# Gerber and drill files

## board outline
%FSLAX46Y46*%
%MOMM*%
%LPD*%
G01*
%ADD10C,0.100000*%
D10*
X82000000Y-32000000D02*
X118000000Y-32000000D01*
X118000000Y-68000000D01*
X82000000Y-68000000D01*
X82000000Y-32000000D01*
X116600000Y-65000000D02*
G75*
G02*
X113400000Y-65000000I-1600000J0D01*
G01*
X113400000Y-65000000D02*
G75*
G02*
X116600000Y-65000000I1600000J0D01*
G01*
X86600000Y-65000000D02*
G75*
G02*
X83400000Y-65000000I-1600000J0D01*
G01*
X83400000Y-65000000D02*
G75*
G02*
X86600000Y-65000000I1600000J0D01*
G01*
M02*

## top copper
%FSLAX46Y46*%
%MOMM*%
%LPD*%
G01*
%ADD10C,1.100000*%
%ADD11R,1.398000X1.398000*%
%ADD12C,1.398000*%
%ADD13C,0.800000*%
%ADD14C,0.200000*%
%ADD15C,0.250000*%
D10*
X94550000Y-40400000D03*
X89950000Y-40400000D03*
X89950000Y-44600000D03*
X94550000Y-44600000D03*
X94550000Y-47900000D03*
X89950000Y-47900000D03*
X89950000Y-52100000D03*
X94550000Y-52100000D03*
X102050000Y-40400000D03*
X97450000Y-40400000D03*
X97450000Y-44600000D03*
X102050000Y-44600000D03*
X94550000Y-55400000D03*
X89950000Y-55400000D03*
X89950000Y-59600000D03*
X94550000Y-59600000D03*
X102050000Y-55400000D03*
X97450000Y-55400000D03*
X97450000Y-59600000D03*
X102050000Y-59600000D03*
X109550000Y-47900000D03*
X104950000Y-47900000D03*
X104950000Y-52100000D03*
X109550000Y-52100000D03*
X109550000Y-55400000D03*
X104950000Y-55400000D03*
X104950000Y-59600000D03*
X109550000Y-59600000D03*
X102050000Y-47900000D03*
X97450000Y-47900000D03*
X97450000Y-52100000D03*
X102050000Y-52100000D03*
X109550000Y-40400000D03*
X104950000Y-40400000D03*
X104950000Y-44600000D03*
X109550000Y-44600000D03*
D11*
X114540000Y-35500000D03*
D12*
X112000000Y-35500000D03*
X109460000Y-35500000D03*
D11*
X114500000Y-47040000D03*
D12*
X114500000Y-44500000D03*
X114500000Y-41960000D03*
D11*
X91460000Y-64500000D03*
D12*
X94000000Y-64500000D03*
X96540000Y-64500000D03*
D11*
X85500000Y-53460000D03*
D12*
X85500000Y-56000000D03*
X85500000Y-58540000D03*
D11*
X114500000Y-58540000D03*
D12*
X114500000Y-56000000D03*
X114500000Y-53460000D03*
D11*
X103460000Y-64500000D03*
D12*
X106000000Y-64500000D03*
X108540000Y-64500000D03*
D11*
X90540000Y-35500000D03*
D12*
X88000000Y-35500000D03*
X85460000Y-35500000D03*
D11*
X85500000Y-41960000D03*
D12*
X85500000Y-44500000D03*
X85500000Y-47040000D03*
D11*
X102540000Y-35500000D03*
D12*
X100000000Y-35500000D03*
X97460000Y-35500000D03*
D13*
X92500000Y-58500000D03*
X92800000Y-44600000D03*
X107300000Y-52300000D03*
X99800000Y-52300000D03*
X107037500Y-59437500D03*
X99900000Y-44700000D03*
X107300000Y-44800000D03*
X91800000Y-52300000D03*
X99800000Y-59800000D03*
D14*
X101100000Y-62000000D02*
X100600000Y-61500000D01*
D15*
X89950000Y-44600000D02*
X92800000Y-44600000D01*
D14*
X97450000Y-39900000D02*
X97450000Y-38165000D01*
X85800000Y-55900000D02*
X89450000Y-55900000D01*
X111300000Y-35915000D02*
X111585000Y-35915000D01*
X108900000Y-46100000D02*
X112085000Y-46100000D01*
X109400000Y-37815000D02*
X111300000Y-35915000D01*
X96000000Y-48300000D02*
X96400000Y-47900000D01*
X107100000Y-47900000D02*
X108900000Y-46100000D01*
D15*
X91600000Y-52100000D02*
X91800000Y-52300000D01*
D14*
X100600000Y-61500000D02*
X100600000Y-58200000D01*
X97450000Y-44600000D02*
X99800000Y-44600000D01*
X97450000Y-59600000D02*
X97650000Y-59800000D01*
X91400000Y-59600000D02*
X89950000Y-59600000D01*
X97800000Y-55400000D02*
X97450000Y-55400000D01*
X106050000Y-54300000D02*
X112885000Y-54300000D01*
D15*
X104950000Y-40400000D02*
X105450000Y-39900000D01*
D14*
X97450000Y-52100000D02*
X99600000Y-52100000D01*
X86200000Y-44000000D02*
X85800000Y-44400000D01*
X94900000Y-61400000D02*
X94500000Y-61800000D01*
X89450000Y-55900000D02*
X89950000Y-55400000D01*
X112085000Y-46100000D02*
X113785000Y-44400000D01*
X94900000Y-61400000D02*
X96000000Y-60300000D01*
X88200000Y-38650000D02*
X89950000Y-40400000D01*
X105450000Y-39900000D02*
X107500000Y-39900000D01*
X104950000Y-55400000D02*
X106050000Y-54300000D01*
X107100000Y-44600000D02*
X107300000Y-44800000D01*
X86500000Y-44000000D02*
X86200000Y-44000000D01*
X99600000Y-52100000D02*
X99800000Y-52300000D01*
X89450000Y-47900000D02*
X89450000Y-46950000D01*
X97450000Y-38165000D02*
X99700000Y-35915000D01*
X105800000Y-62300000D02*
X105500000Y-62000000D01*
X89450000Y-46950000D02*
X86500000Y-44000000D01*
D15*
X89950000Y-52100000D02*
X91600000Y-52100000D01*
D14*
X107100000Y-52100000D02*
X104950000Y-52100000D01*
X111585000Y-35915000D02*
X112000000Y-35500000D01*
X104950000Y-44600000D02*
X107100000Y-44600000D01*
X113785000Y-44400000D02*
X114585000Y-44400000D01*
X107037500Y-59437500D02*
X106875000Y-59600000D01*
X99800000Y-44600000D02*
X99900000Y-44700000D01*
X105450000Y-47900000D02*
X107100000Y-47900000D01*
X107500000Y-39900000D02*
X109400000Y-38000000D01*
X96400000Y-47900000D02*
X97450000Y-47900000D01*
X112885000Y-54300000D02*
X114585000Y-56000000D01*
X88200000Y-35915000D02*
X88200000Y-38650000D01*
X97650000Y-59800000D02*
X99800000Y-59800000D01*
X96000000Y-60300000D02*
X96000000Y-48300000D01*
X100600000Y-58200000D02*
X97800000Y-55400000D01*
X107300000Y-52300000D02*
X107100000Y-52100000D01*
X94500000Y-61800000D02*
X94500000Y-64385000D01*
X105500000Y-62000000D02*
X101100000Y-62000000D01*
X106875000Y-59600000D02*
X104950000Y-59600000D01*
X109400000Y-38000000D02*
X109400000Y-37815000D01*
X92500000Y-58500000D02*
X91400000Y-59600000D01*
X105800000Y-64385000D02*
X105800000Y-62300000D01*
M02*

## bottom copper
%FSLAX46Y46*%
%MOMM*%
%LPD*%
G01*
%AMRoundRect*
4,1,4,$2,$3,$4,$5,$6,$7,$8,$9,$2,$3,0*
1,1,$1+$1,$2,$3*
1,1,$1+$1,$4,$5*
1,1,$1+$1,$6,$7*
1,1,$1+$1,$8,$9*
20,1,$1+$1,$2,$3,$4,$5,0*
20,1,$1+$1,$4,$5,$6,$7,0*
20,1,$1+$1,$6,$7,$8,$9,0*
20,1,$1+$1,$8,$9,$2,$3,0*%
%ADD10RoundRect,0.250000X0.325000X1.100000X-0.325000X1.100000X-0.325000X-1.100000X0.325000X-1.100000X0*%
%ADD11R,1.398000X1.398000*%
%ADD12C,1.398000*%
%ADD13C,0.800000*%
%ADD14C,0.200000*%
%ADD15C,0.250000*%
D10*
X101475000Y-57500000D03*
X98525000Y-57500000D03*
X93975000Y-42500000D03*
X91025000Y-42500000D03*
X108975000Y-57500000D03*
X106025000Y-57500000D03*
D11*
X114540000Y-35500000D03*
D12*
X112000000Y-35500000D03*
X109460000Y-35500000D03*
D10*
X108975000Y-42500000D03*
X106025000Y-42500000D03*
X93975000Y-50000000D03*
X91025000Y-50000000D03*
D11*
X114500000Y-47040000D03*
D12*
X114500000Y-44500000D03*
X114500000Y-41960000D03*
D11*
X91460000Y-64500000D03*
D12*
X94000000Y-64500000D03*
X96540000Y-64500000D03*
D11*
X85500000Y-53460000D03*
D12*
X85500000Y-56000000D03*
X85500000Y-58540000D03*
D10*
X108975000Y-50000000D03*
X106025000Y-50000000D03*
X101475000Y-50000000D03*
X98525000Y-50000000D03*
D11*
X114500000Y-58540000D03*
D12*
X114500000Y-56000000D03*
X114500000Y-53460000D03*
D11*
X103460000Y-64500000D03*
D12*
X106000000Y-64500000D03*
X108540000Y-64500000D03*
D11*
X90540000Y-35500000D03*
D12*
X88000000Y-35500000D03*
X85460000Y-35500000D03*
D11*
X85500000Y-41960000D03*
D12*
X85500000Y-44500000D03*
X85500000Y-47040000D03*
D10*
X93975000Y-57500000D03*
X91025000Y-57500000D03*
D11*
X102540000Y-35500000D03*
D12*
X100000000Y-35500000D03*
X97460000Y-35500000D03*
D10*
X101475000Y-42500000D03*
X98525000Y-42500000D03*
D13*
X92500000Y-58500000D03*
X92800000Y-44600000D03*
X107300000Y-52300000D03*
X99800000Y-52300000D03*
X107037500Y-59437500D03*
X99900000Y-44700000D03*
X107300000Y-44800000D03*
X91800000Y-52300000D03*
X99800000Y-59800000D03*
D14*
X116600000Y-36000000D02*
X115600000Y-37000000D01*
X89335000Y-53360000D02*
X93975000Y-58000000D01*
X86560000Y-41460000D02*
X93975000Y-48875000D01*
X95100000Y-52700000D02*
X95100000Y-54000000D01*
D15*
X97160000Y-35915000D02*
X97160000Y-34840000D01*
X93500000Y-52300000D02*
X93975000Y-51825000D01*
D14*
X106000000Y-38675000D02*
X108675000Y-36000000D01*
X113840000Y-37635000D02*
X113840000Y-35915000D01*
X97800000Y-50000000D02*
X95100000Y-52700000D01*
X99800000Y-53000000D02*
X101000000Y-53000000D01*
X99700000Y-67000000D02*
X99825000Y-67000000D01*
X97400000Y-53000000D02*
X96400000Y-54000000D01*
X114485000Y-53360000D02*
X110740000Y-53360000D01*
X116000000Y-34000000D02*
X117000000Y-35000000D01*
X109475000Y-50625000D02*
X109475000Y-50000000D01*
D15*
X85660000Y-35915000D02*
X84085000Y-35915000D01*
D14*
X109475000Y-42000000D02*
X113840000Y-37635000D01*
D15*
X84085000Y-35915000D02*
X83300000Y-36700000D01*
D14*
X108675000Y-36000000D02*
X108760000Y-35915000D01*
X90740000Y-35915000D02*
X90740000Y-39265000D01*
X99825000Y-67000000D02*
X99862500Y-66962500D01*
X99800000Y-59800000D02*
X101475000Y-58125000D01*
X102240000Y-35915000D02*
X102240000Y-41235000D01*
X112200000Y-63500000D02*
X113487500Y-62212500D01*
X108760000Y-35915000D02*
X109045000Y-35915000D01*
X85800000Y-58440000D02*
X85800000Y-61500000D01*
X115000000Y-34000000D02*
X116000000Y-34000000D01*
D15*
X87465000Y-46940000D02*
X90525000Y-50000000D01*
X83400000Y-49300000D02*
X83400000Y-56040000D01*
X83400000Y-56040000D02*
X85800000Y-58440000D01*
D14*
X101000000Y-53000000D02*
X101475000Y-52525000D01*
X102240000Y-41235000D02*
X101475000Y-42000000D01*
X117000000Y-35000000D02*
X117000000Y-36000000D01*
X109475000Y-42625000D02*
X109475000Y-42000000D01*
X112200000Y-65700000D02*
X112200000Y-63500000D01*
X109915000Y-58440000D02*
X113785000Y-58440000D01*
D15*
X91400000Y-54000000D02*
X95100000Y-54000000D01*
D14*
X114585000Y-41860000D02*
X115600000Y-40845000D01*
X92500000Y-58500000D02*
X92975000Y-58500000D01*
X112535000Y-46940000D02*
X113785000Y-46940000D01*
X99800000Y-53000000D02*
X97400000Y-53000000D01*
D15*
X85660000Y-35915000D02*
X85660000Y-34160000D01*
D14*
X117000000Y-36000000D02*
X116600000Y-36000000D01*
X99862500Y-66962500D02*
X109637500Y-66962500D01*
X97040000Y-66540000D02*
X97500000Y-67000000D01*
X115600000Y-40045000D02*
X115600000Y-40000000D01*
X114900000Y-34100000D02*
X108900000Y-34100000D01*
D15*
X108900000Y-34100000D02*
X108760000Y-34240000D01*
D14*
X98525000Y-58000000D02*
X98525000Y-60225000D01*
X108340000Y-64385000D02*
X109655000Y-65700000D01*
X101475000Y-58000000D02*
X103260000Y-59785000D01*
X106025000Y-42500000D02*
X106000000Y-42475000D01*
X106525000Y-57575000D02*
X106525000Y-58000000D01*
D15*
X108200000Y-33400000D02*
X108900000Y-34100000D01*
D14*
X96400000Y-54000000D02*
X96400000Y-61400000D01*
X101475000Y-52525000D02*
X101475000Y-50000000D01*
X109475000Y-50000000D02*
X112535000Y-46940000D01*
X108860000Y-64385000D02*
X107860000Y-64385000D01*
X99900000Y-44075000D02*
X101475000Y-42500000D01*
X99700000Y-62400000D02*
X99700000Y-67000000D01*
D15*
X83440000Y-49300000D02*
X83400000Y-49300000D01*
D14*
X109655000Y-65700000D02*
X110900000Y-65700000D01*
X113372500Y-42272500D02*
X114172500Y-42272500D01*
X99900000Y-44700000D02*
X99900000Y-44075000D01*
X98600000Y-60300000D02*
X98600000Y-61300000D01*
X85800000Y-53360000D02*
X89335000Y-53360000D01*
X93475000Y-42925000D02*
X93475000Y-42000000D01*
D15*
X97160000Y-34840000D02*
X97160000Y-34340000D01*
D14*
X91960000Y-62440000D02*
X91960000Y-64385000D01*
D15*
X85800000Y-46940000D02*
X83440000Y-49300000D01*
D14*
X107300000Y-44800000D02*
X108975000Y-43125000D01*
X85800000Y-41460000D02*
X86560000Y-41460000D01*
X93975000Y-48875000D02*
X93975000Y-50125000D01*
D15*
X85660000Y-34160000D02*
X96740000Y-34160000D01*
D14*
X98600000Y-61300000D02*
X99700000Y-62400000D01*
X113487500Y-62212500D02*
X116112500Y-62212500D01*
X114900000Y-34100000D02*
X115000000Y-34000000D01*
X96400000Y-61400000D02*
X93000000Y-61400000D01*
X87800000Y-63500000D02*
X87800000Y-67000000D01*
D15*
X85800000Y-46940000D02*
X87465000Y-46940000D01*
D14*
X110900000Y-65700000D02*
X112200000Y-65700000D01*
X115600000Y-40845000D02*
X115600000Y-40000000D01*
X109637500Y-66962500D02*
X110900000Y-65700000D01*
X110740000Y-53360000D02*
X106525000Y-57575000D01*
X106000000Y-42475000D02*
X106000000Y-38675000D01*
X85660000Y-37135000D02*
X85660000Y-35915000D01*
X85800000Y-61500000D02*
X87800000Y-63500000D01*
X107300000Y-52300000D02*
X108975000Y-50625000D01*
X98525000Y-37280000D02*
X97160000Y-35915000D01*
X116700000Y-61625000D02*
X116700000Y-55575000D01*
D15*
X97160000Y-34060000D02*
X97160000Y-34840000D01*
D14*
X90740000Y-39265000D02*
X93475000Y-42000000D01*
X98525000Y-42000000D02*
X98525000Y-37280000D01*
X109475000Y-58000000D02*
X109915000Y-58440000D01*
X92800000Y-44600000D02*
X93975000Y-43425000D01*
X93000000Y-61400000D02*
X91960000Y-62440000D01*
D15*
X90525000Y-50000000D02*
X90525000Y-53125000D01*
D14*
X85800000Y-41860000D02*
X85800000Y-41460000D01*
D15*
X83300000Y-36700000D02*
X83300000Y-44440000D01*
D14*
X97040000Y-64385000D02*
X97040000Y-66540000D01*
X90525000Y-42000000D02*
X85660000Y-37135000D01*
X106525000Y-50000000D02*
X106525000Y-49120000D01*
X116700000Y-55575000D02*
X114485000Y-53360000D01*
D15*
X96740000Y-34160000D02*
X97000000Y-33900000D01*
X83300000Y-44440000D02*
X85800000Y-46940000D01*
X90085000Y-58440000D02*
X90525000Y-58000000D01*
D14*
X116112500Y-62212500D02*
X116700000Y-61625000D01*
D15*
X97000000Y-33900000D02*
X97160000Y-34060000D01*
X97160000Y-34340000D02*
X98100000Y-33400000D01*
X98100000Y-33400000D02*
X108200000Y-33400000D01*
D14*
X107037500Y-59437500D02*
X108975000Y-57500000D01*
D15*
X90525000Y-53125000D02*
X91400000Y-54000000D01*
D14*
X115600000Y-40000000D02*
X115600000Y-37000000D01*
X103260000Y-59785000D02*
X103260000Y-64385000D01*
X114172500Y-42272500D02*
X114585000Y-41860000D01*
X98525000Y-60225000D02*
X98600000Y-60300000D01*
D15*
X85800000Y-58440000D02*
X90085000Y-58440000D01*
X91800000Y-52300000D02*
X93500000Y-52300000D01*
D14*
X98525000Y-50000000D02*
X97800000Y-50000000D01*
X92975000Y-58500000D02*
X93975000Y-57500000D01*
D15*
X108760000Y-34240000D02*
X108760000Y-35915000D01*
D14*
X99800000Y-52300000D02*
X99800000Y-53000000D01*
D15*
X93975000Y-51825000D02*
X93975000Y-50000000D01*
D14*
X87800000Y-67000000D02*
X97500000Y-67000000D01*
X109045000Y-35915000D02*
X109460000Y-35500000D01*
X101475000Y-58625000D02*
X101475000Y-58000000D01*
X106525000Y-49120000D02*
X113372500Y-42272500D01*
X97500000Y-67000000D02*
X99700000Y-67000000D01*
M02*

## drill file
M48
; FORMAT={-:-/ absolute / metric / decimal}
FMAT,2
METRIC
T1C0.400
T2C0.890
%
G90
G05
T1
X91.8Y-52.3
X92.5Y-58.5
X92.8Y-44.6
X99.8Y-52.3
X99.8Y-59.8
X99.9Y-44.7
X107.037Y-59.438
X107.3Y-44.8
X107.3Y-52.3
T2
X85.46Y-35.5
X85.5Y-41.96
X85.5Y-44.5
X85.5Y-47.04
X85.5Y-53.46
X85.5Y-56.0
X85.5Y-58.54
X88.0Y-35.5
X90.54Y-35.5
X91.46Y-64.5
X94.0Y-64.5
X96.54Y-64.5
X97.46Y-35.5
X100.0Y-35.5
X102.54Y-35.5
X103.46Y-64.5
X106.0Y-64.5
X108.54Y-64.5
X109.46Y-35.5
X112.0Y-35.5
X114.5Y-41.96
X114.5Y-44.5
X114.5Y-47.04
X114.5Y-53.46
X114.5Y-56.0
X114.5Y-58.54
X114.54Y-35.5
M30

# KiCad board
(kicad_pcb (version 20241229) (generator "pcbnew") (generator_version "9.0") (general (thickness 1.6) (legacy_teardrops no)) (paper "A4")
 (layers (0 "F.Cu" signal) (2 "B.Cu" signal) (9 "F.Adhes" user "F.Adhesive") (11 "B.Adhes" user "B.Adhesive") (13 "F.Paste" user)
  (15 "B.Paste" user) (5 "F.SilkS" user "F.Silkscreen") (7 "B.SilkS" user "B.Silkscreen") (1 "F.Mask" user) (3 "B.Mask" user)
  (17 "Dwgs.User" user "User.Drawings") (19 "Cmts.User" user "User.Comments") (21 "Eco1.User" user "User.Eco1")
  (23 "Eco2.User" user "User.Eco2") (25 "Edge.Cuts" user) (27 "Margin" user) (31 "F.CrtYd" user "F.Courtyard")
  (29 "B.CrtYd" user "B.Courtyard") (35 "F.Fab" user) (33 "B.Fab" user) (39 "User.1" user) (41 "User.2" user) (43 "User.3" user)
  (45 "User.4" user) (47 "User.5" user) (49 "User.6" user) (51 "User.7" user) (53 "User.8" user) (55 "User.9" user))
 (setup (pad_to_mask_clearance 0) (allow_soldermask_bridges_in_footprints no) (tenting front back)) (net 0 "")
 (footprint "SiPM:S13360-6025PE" (layer "F.Cu") (at 92.5 42.5)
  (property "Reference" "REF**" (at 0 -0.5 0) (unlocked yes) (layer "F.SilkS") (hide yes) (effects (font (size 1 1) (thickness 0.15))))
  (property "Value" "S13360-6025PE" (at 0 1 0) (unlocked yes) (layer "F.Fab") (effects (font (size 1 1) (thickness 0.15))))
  (pad "1" smd circle (at 2.05 -2.1) (size 1.1 1.1) (layers "F.Cu" "F.Mask" "F.Paste"))
  (pad "2" smd circle (at -2.55 -2.1) (size 1.1 1.1) (layers "F.Cu" "F.Mask" "F.Paste"))
  (pad "3" smd circle (at -2.55 2.1) (size 1.1 1.1) (layers "F.Cu" "F.Mask" "F.Paste"))
  (pad "4" smd circle (at 2.05 2.1) (size 1.1 1.1) (layers "F.Cu" "F.Mask" "F.Paste")))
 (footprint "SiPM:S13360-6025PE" (layer "F.Cu") (at 92.5 50)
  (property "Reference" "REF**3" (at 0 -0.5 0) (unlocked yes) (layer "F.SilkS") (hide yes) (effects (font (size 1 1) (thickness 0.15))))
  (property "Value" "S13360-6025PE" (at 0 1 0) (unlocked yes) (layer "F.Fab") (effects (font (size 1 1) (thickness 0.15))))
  (pad "1" smd circle (at 2.05 -2.1) (size 1.1 1.1) (layers "F.Cu" "F.Mask" "F.Paste"))
  (pad "2" smd circle (at -2.55 -2.1) (size 1.1 1.1) (layers "F.Cu" "F.Mask" "F.Paste"))
  (pad "3" smd circle (at -2.55 2.1) (size 1.1 1.1) (layers "F.Cu" "F.Mask" "F.Paste"))
  (pad "4" smd circle (at 2.05 2.1) (size 1.1 1.1) (layers "F.Cu" "F.Mask" "F.Paste")))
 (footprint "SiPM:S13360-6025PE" (layer "F.Cu") (at 100 42.5)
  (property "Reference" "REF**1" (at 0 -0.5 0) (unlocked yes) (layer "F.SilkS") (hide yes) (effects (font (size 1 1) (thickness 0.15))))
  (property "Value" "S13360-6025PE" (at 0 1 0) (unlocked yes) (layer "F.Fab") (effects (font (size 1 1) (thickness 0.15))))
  (pad "1" smd circle (at 2.05 -2.1) (size 1.1 1.1) (layers "F.Cu" "F.Mask" "F.Paste"))
  (pad "2" smd circle (at -2.55 -2.1) (size 1.1 1.1) (layers "F.Cu" "F.Mask" "F.Paste"))
  (pad "3" smd circle (at -2.55 2.1) (size 1.1 1.1) (layers "F.Cu" "F.Mask" "F.Paste"))
  (pad "4" smd circle (at 2.05 2.1) (size 1.1 1.1) (layers "F.Cu" "F.Mask" "F.Paste")))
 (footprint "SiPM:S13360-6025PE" (layer "F.Cu") (at 92.5 57.5)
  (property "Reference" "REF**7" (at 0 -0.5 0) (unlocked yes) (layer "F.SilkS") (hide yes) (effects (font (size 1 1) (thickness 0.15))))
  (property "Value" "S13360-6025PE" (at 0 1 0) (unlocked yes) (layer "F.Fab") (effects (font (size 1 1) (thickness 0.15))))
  (pad "1" smd circle (at 2.05 -2.1) (size 1.1 1.1) (layers "F.Cu" "F.Mask" "F.Paste"))
  (pad "2" smd circle (at -2.55 -2.1) (size 1.1 1.1) (layers "F.Cu" "F.Mask" "F.Paste"))
  (pad "3" smd circle (at -2.55 2.1) (size 1.1 1.1) (layers "F.Cu" "F.Mask" "F.Paste"))
  (pad "4" smd circle (at 2.05 2.1) (size 1.1 1.1) (layers "F.Cu" "F.Mask" "F.Paste")))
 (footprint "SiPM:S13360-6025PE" (layer "F.Cu") (at 100 57.5)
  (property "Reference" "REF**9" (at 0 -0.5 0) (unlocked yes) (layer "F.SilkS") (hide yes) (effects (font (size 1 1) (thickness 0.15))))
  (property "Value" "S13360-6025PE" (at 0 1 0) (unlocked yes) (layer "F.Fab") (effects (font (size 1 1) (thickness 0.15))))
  (pad "1" smd circle (at 2.05 -2.1) (size 1.1 1.1) (layers "F.Cu" "F.Mask" "F.Paste"))
  (pad "2" smd circle (at -2.55 -2.1) (size 1.1 1.1) (layers "F.Cu" "F.Mask" "F.Paste"))
  (pad "3" smd circle (at -2.55 2.1) (size 1.1 1.1) (layers "F.Cu" "F.Mask" "F.Paste"))
  (pad "4" smd circle (at 2.05 2.1) (size 1.1 1.1) (layers "F.Cu" "F.Mask" "F.Paste")))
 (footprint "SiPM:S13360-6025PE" (layer "F.Cu") (at 107.5 50)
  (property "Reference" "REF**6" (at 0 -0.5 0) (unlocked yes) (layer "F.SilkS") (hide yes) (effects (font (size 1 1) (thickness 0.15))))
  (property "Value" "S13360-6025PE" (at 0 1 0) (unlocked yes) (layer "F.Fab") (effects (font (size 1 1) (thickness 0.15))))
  (pad "1" smd circle (at 2.05 -2.1) (size 1.1 1.1) (layers "F.Cu" "F.Mask" "F.Paste"))
  (pad "2" smd circle (at -2.55 -2.1) (size 1.1 1.1) (layers "F.Cu" "F.Mask" "F.Paste"))
  (pad "3" smd circle (at -2.55 2.1) (size 1.1 1.1) (layers "F.Cu" "F.Mask" "F.Paste"))
  (pad "4" smd circle (at 2.05 2.1) (size 1.1 1.1) (layers "F.Cu" "F.Mask" "F.Paste")))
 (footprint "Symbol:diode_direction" (layer "F.Cu") (at 87.3 41.8 90)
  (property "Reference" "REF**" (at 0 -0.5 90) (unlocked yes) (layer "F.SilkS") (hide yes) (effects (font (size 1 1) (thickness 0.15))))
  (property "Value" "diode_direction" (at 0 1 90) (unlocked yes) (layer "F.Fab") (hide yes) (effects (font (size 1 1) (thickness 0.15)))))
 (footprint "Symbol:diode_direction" (layer "F.Cu") (at 87.3 49.8 90)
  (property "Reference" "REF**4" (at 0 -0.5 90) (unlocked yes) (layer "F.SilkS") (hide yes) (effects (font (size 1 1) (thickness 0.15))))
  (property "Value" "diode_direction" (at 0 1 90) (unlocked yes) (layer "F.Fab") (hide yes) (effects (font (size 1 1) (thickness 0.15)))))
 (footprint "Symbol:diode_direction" (layer "F.Cu") (at 87.3 57.8 90)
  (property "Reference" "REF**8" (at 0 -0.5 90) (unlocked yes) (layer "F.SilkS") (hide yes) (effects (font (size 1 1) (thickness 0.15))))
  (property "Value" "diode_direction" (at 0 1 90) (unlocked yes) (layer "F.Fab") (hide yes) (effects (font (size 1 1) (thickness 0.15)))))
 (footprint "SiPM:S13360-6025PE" (layer "F.Cu") (at 107.5 57.5)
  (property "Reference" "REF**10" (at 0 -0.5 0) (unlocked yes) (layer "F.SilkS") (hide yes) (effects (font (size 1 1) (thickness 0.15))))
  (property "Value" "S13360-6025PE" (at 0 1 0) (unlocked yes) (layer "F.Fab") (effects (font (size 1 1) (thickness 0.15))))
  (pad "1" smd circle (at 2.05 -2.1) (size 1.1 1.1) (layers "F.Cu" "F.Mask" "F.Paste"))
  (pad "2" smd circle (at -2.55 -2.1) (size 1.1 1.1) (layers "F.Cu" "F.Mask" "F.Paste"))
  (pad "3" smd circle (at -2.55 2.1) (size 1.1 1.1) (layers "F.Cu" "F.Mask" "F.Paste"))
  (pad "4" smd circle (at 2.05 2.1) (size 1.1 1.1) (layers "F.Cu" "F.Mask" "F.Paste")))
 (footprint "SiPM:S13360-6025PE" (layer "F.Cu") (at 100 50)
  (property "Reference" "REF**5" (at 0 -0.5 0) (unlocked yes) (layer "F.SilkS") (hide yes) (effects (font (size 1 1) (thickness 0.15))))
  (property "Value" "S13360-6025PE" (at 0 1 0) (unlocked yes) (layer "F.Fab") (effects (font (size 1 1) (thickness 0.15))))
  (pad "1" smd circle (at 2.05 -2.1) (size 1.1 1.1) (layers "F.Cu" "F.Mask" "F.Paste"))
  (pad "2" smd circle (at -2.55 -2.1) (size 1.1 1.1) (layers "F.Cu" "F.Mask" "F.Paste"))
  (pad "3" smd circle (at -2.55 2.1) (size 1.1 1.1) (layers "F.Cu" "F.Mask" "F.Paste"))
  (pad "4" smd circle (at 2.05 2.1) (size 1.1 1.1) (layers "F.Cu" "F.Mask" "F.Paste")))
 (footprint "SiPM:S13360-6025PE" (layer "F.Cu") (at 107.5 42.5)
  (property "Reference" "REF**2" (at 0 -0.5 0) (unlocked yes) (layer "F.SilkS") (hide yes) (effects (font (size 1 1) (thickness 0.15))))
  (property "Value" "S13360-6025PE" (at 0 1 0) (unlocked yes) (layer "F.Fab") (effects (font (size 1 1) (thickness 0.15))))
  (pad "1" smd circle (at 2.05 -2.1) (size 1.1 1.1) (layers "F.Cu" "F.Mask" "F.Paste"))
  (pad "2" smd circle (at -2.55 -2.1) (size 1.1 1.1) (layers "F.Cu" "F.Mask" "F.Paste"))
  (pad "3" smd circle (at -2.55 2.1) (size 1.1 1.1) (layers "F.Cu" "F.Mask" "F.Paste"))
  (pad "4" smd circle (at 2.05 2.1) (size 1.1 1.1) (layers "F.Cu" "F.Mask" "F.Paste")))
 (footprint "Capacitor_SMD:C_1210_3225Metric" (layer "B.Cu") (at 100 57.5 180)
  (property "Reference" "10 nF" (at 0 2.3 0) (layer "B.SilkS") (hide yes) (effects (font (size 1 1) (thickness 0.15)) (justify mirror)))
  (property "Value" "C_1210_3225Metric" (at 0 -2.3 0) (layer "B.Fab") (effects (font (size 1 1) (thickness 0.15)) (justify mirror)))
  (pad "1" smd roundrect (at -1.475 0 180) (size 1.15 2.7) (layers "B.Cu" "B.Mask" "B.Paste") (roundrect_rratio 0.2173913043))
  (pad "2" smd roundrect (at 1.475 0 180) (size 1.15 2.7) (layers "B.Cu" "B.Mask" "B.Paste") (roundrect_rratio 0.2173913043)))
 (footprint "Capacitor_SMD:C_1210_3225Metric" (layer "B.Cu") (at 92.5 42.5 180)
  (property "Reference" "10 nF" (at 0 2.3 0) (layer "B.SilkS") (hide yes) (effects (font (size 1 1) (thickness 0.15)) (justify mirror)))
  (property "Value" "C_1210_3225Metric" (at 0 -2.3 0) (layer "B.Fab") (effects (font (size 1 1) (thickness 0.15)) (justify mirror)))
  (pad "1" smd roundrect (at -1.475 0 180) (size 1.15 2.7) (layers "B.Cu" "B.Mask" "B.Paste") (roundrect_rratio 0.2173913043))
  (pad "2" smd roundrect (at 1.475 0 180) (size 1.15 2.7) (layers "B.Cu" "B.Mask" "B.Paste") (roundrect_rratio 0.2173913043)))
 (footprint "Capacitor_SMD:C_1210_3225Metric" (layer "B.Cu") (at 107.5 57.5 180)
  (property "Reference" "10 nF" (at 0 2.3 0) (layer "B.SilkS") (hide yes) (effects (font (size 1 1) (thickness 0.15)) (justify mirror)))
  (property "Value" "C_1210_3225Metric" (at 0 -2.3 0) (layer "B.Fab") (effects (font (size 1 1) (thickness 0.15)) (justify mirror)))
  (pad "1" smd roundrect (at -1.475 0 180) (size 1.15 2.7) (layers "B.Cu" "B.Mask" "B.Paste") (roundrect_rratio 0.2173913043))
  (pad "2" smd roundrect (at 1.475 0 180) (size 1.15 2.7) (layers "B.Cu" "B.Mask" "B.Paste") (roundrect_rratio 0.2173913043)))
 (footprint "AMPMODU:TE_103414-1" (layer "B.Cu") (at 112 35.5 180)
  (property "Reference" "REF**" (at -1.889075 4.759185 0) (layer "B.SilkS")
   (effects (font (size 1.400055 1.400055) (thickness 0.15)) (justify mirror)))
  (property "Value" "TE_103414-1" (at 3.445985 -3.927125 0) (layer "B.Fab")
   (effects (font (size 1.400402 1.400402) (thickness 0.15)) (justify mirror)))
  (pad "1" thru_hole rect (at -2.54 0 180) (size 1.398 1.398) (drill 0.89) (layers "*.Cu" "*.Mask") (remove_unused_layers no)
   (solder_mask_margin 0.102))
  (pad "2" thru_hole circle (at 0 0 180) (size 1.398 1.398) (drill 0.89) (layers "*.Cu" "*.Mask") (remove_unused_layers no)
   (solder_mask_margin 0.102))
  (pad "3" thru_hole circle (at 2.54 0 180) (size 1.398 1.398) (drill 0.89) (layers "*.Cu" "*.Mask") (remove_unused_layers no)
   (solder_mask_margin 0.102)))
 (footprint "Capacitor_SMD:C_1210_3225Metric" (layer "B.Cu") (at 107.5 42.5 180)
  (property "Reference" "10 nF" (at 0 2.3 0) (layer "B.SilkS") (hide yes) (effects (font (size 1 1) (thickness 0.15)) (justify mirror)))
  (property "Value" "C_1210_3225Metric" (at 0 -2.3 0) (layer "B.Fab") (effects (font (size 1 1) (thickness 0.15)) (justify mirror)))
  (pad "1" smd roundrect (at -1.475 0 180) (size 1.15 2.7) (layers "B.Cu" "B.Mask" "B.Paste") (roundrect_rratio 0.2173913043))
  (pad "2" smd roundrect (at 1.475 0 180) (size 1.15 2.7) (layers "B.Cu" "B.Mask" "B.Paste") (roundrect_rratio 0.2173913043)))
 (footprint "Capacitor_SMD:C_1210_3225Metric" (layer "B.Cu") (at 92.5 50 180)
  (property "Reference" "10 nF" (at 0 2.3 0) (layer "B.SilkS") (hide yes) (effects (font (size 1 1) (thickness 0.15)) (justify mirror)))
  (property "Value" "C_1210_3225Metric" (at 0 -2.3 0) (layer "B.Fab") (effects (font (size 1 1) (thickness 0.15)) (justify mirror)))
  (pad "1" smd roundrect (at -1.475 0 180) (size 1.15 2.7) (layers "B.Cu" "B.Mask" "B.Paste") (roundrect_rratio 0.2173913043))
  (pad "2" smd roundrect (at 1.475 0 180) (size 1.15 2.7) (layers "B.Cu" "B.Mask" "B.Paste") (roundrect_rratio 0.2173913043)))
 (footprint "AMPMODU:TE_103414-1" (layer "B.Cu") (at 114.5 44.5 90)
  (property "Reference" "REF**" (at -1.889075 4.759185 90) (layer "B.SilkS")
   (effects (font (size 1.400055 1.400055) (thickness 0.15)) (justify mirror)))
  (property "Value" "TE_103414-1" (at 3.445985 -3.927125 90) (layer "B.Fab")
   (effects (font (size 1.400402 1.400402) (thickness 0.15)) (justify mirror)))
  (pad "1" thru_hole rect (at -2.54 0 90) (size 1.398 1.398) (drill 0.89) (layers "*.Cu" "*.Mask") (remove_unused_layers no)
   (solder_mask_margin 0.102))
  (pad "2" thru_hole circle (at 0 0 90) (size 1.398 1.398) (drill 0.89) (layers "*.Cu" "*.Mask") (remove_unused_layers no)
   (solder_mask_margin 0.102))
  (pad "3" thru_hole circle (at 2.54 0 90) (size 1.398 1.398) (drill 0.89) (layers "*.Cu" "*.Mask") (remove_unused_layers no)
   (solder_mask_margin 0.102)))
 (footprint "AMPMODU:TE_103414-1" (layer "B.Cu") (at 94 64.5)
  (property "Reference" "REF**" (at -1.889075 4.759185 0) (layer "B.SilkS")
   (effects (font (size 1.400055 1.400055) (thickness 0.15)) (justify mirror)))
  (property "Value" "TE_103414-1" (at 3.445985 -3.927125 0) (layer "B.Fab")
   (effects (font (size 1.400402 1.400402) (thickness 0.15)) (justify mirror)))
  (pad "1" thru_hole rect (at -2.54 0) (size 1.398 1.398) (drill 0.89) (layers "*.Cu" "*.Mask") (remove_unused_layers no)
   (solder_mask_margin 0.102))
  (pad "2" thru_hole circle (at 0 0) (size 1.398 1.398) (drill 0.89) (layers "*.Cu" "*.Mask") (remove_unused_layers no)
   (solder_mask_margin 0.102))
  (pad "3" thru_hole circle (at 2.54 0) (size 1.398 1.398) (drill 0.89) (layers "*.Cu" "*.Mask") (remove_unused_layers no)
   (solder_mask_margin 0.102)))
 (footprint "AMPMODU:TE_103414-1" (layer "B.Cu") (at 85.5 56 -90)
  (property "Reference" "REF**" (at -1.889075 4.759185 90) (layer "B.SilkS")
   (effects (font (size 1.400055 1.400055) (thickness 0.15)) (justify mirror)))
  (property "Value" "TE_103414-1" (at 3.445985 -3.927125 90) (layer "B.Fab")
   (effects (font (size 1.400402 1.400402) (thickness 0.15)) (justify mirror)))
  (pad "1" thru_hole rect (at -2.54 0 270) (size 1.398 1.398) (drill 0.89) (layers "*.Cu" "*.Mask") (remove_unused_layers no)
   (solder_mask_margin 0.102))
  (pad "2" thru_hole circle (at 0 0 270) (size 1.398 1.398) (drill 0.89) (layers "*.Cu" "*.Mask") (remove_unused_layers no)
   (solder_mask_margin 0.102))
  (pad "3" thru_hole circle (at 2.54 0 270) (size 1.398 1.398) (drill 0.89) (layers "*.Cu" "*.Mask") (remove_unused_layers no)
   (solder_mask_margin 0.102)))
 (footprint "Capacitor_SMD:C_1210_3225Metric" (layer "B.Cu") (at 107.5 50 180)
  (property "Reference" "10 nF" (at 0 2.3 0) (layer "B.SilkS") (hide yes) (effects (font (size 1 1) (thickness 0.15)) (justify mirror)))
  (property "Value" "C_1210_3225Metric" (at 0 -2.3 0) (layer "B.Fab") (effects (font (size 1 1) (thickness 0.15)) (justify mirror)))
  (pad "1" smd roundrect (at -1.475 0 180) (size 1.15 2.7) (layers "B.Cu" "B.Mask" "B.Paste") (roundrect_rratio 0.2173913043))
  (pad "2" smd roundrect (at 1.475 0 180) (size 1.15 2.7) (layers "B.Cu" "B.Mask" "B.Paste") (roundrect_rratio 0.2173913043)))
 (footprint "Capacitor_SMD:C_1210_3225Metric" (layer "B.Cu") (at 100 50 180)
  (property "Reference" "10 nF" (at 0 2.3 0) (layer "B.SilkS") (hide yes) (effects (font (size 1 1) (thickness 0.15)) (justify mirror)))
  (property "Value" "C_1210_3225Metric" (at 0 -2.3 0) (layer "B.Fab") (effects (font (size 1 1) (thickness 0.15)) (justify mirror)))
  (pad "1" smd roundrect (at -1.475 0 180) (size 1.15 2.7) (layers "B.Cu" "B.Mask" "B.Paste") (roundrect_rratio 0.2173913043))
  (pad "2" smd roundrect (at 1.475 0 180) (size 1.15 2.7) (layers "B.Cu" "B.Mask" "B.Paste") (roundrect_rratio 0.2173913043)))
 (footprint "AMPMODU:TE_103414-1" (layer "B.Cu") (at 114.5 56 90)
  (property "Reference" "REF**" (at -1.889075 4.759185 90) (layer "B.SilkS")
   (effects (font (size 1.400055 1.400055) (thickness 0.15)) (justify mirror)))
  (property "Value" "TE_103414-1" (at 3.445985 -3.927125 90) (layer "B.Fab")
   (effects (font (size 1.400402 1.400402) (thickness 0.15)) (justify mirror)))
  (pad "1" thru_hole rect (at -2.54 0 90) (size 1.398 1.398) (drill 0.89) (layers "*.Cu" "*.Mask") (remove_unused_layers no)
   (solder_mask_margin 0.102))
  (pad "2" thru_hole circle (at 0 0 90) (size 1.398 1.398) (drill 0.89) (layers "*.Cu" "*.Mask") (remove_unused_layers no)
   (solder_mask_margin 0.102))
  (pad "3" thru_hole circle (at 2.54 0 90) (size 1.398 1.398) (drill 0.89) (layers "*.Cu" "*.Mask") (remove_unused_layers no)
   (solder_mask_margin 0.102)))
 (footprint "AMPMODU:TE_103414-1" (layer "B.Cu") (at 106 64.5)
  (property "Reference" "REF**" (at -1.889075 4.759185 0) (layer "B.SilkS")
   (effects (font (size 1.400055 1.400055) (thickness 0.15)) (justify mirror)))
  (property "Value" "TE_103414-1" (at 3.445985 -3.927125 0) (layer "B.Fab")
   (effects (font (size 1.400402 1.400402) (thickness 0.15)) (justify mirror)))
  (pad "1" thru_hole rect (at -2.54 0) (size 1.398 1.398) (drill 0.89) (layers "*.Cu" "*.Mask") (remove_unused_layers no)
   (solder_mask_margin 0.102))
  (pad "2" thru_hole circle (at 0 0) (size 1.398 1.398) (drill 0.89) (layers "*.Cu" "*.Mask") (remove_unused_layers no)
   (solder_mask_margin 0.102))
  (pad "3" thru_hole circle (at 2.54 0) (size 1.398 1.398) (drill 0.89) (layers "*.Cu" "*.Mask") (remove_unused_layers no)
   (solder_mask_margin 0.102)))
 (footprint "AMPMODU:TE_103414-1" (layer "B.Cu") (at 88 35.5 180)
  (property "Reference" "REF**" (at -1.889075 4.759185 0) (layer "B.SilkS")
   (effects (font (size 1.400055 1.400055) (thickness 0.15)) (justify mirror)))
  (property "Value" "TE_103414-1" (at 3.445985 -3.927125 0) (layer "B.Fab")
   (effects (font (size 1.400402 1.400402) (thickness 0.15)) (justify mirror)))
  (pad "1" thru_hole rect (at -2.54 0 180) (size 1.398 1.398) (drill 0.89) (layers "*.Cu" "*.Mask") (remove_unused_layers no)
   (solder_mask_margin 0.102))
  (pad "2" thru_hole circle (at 0 0 180) (size 1.398 1.398) (drill 0.89) (layers "*.Cu" "*.Mask") (remove_unused_layers no)
   (solder_mask_margin 0.102))
  (pad "3" thru_hole circle (at 2.54 0 180) (size 1.398 1.398) (drill 0.89) (layers "*.Cu" "*.Mask") (remove_unused_layers no)
   (solder_mask_margin 0.102)))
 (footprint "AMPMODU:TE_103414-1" (layer "B.Cu") (at 85.5 44.5 -90)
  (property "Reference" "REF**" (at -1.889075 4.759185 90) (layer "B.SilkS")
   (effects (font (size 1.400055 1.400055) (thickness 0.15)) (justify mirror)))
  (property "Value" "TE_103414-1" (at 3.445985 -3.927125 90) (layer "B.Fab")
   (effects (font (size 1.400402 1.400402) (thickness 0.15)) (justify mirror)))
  (pad "1" thru_hole rect (at -2.54 0 270) (size 1.398 1.398) (drill 0.89) (layers "*.Cu" "*.Mask") (remove_unused_layers no)
   (solder_mask_margin 0.102))
  (pad "2" thru_hole circle (at 0 0 270) (size 1.398 1.398) (drill 0.89) (layers "*.Cu" "*.Mask") (remove_unused_layers no)
   (solder_mask_margin 0.102))
  (pad "3" thru_hole circle (at 2.54 0 270) (size 1.398 1.398) (drill 0.89) (layers "*.Cu" "*.Mask") (remove_unused_layers no)
   (solder_mask_margin 0.102)))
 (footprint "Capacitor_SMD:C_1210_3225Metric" (layer "B.Cu") (at 92.5 57.5 180)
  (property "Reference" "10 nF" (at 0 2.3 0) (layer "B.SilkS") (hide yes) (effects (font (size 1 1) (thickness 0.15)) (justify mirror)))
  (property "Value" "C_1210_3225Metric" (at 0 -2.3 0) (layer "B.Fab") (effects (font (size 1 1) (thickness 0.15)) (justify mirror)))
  (pad "1" smd roundrect (at -1.475 0 180) (size 1.15 2.7) (layers "B.Cu" "B.Mask" "B.Paste") (roundrect_rratio 0.2173913043))
  (pad "2" smd roundrect (at 1.475 0 180) (size 1.15 2.7) (layers "B.Cu" "B.Mask" "B.Paste") (roundrect_rratio 0.2173913043)))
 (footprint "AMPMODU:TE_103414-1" (layer "B.Cu") (at 100 35.5 180)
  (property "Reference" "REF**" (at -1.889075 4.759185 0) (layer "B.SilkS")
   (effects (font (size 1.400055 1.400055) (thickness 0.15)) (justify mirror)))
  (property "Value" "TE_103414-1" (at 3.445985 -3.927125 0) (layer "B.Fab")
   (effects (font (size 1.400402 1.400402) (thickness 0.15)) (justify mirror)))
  (pad "1" thru_hole rect (at -2.54 0 180) (size 1.398 1.398) (drill 0.89) (layers "*.Cu" "*.Mask") (remove_unused_layers no)
   (solder_mask_margin 0.102))
  (pad "2" thru_hole circle (at 0 0 180) (size 1.398 1.398) (drill 0.89) (layers "*.Cu" "*.Mask") (remove_unused_layers no)
   (solder_mask_margin 0.102))
  (pad "3" thru_hole circle (at 2.54 0 180) (size 1.398 1.398) (drill 0.89) (layers "*.Cu" "*.Mask") (remove_unused_layers no)
   (solder_mask_margin 0.102)))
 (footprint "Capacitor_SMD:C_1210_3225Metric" (layer "B.Cu") (at 100 42.5 180)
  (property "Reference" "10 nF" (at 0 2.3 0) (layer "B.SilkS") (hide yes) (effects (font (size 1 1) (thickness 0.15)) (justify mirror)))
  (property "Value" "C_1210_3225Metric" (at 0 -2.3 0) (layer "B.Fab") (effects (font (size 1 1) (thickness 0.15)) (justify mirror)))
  (pad "1" smd roundrect (at -1.475 0 180) (size 1.15 2.7) (layers "B.Cu" "B.Mask" "B.Paste") (roundrect_rratio 0.2173913043))
  (pad "2" smd roundrect (at 1.475 0 180) (size 1.15 2.7) (layers "B.Cu" "B.Mask" "B.Paste") (roundrect_rratio 0.2173913043)))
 (gr_rect (start 82 32) (end 118 68) (stroke (width 0.1) (type solid)) (fill no) (layer "Edge.Cuts"))
 (gr_circle (center 115 65) (end 115 63.4) (stroke (width 0.1) (type solid)) (fill no) (layer "Edge.Cuts"))
 (gr_circle (center 85 65) (end 85 63.4) (stroke (width 0.1) (type solid)) (fill no) (layer "Edge.Cuts"))
 (segment (start 101.1 62) (end 100.6 61.5) (width 0.2) (layer "F.Cu") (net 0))
 (segment (start 89.95 44.6) (end 92.8 44.6) (width 0.25) (layer "F.Cu") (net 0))
 (segment (start 97.45 39.9) (end 97.45 38.165) (width 0.2) (layer "F.Cu") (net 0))
 (segment (start 85.8 55.9) (end 89.45 55.9) (width 0.2) (layer "F.Cu") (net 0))
 (segment (start 111.3 35.915) (end 111.585 35.915) (width 0.2) (layer "F.Cu") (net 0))
 (segment (start 108.9 46.1) (end 112.085 46.1) (width 0.2) (layer "F.Cu") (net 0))
 (segment (start 109.4 37.815) (end 111.3 35.915) (width 0.2) (layer "F.Cu") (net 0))
 (segment (start 96 48.3) (end 96.4 47.9) (width 0.2) (layer "F.Cu") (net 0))
 (segment (start 107.1 47.9) (end 108.9 46.1) (width 0.2) (layer "F.Cu") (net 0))
 (segment (start 91.6 52.1) (end 91.8 52.3) (width 0.25) (layer "F.Cu") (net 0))
 (segment (start 100.6 61.5) (end 100.6 58.2) (width 0.2) (layer "F.Cu") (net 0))
 (segment (start 97.45 44.6) (end 99.8 44.6) (width 0.2) (layer "F.Cu") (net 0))
 (segment (start 97.45 59.6) (end 97.65 59.8) (width 0.2) (layer "F.Cu") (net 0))
 (segment (start 91.4 59.6) (end 89.95 59.6) (width 0.2) (layer "F.Cu") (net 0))
 (segment (start 97.8 55.4) (end 97.45 55.4) (width 0.2) (layer "F.Cu") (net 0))
 (segment (start 106.05 54.3) (end 112.885 54.3) (width 0.2) (layer "F.Cu") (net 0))
 (segment (start 104.95 40.4) (end 105.45 39.9) (width 0.25) (layer "F.Cu") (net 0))
 (segment (start 97.45 52.1) (end 99.6 52.1) (width 0.2) (layer "F.Cu") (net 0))
 (segment (start 86.2 44) (end 85.8 44.4) (width 0.2) (layer "F.Cu") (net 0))
 (segment (start 94.9 61.4) (end 94.5 61.8) (width 0.2) (layer "F.Cu") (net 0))
 (segment (start 89.45 55.9) (end 89.95 55.4) (width 0.2) (layer "F.Cu") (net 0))
 (segment (start 112.085 46.1) (end 113.785 44.4) (width 0.2) (layer "F.Cu") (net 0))
 (segment (start 94.9 61.4) (end 96 60.3) (width 0.2) (layer "F.Cu") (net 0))
 (segment (start 88.2 38.65) (end 89.95 40.4) (width 0.2) (layer "F.Cu") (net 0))
 (segment (start 105.45 39.9) (end 107.5 39.9) (width 0.2) (layer "F.Cu") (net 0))
 (segment (start 104.95 55.4) (end 106.05 54.3) (width 0.2) (layer "F.Cu") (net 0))
 (segment (start 107.1 44.6) (end 107.3 44.8) (width 0.2) (layer "F.Cu") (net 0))
 (segment (start 86.5 44) (end 86.2 44) (width 0.2) (layer "F.Cu") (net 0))
 (segment (start 99.6 52.1) (end 99.8 52.3) (width 0.2) (layer "F.Cu") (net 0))
 (segment (start 89.45 47.9) (end 89.45 46.95) (width 0.2) (layer "F.Cu") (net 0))
 (segment (start 97.45 38.165) (end 99.7 35.915) (width 0.2) (layer "F.Cu") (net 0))
 (segment (start 105.8 62.3) (end 105.5 62) (width 0.2) (layer "F.Cu") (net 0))
 (segment (start 89.45 46.95) (end 86.5 44) (width 0.2) (layer "F.Cu") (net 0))
 (segment (start 89.95 52.1) (end 91.6 52.1) (width 0.25) (layer "F.Cu") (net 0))
 (segment (start 107.1 52.1) (end 104.95 52.1) (width 0.2) (layer "F.Cu") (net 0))
 (segment (start 111.585 35.915) (end 112 35.5) (width 0.2) (layer "F.Cu") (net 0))
 (segment (start 104.95 44.6) (end 107.1 44.6) (width 0.2) (layer "F.Cu") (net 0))
 (segment (start 113.785 44.4) (end 114.585 44.4) (width 0.2) (layer "F.Cu") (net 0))
 (segment (start 107.0375 59.4375) (end 106.875 59.6) (width 0.2) (layer "F.Cu") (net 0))
 (segment (start 99.8 44.6) (end 99.9 44.7) (width 0.2) (layer "F.Cu") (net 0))
 (segment (start 105.45 47.9) (end 107.1 47.9) (width 0.2) (layer "F.Cu") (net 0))
 (segment (start 107.5 39.9) (end 109.4 38) (width 0.2) (layer "F.Cu") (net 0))
 (segment (start 96.4 47.9) (end 97.45 47.9) (width 0.2) (layer "F.Cu") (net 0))
 (segment (start 112.885 54.3) (end 114.585 56) (width 0.2) (layer "F.Cu") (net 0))
 (segment (start 88.2 35.915) (end 88.2 38.65) (width 0.2) (layer "F.Cu") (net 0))
 (segment (start 97.65 59.8) (end 99.8 59.8) (width 0.2) (layer "F.Cu") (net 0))
 (segment (start 96 60.3) (end 96 48.3) (width 0.2) (layer "F.Cu") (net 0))
 (segment (start 100.6 58.2) (end 97.8 55.4) (width 0.2) (layer "F.Cu") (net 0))
 (segment (start 107.3 52.3) (end 107.1 52.1) (width 0.2) (layer "F.Cu") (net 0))
 (segment (start 94.5 61.8) (end 94.5 64.385) (width 0.2) (layer "F.Cu") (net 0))
 (segment (start 105.5 62) (end 101.1 62) (width 0.2) (layer "F.Cu") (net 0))
 (segment (start 106.875 59.6) (end 104.95 59.6) (width 0.2) (layer "F.Cu") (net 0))
 (segment (start 109.4 38) (end 109.4 37.815) (width 0.2) (layer "F.Cu") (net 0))
 (segment (start 92.5 58.5) (end 91.4 59.6) (width 0.2) (layer "F.Cu") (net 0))
 (segment (start 105.8 64.385) (end 105.8 62.3) (width 0.2) (layer "F.Cu") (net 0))
 (via (at 92.5 58.5) (size 0.8) (drill 0.4) (layers "F.Cu" "B.Cu") (free yes) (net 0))
 (via (at 92.8 44.6) (size 0.8) (drill 0.4) (layers "F.Cu" "B.Cu") (free yes) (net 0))
 (via (at 107.3 52.3) (size 0.8) (drill 0.4) (layers "F.Cu" "B.Cu") (free yes) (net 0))
 (via (at 99.8 52.3) (size 0.8) (drill 0.4) (layers "F.Cu" "B.Cu") (free yes) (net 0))
 (via (at 107.0375 59.4375) (size 0.8) (drill 0.4) (layers "F.Cu" "B.Cu") (free yes) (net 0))
 (via (at 99.9 44.7) (size 0.8) (drill 0.4) (layers "F.Cu" "B.Cu") (free yes) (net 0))
 (via (at 107.3 44.8) (size 0.8) (drill 0.4) (layers "F.Cu" "B.Cu") (free yes) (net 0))
 (via (at 91.8 52.3) (size 0.8) (drill 0.4) (layers "F.Cu" "B.Cu") (free yes) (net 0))
 (via (at 99.8 59.8) (size 0.8) (drill 0.4) (layers "F.Cu" "B.Cu") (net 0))
 (segment (start 116.6 36) (end 115.6 37) (width 0.2) (layer "B.Cu") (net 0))
 (segment (start 89.335 53.36) (end 93.975 58) (width 0.2) (layer "B.Cu") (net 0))
 (segment (start 86.56 41.46) (end 93.975 48.875) (width 0.2) (layer "B.Cu") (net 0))
 (segment (start 95.1 52.7) (end 95.1 54) (width 0.2) (layer "B.Cu") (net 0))
 (segment (start 97.16 35.915) (end 97.16 34.84) (width 0.25) (layer "B.Cu") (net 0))
 (segment (start 93.5 52.3) (end 93.975 51.825) (width 0.25) (layer "B.Cu") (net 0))
 (segment (start 106 38.675) (end 108.675 36) (width 0.2) (layer "B.Cu") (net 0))
 (segment (start 113.84 37.635) (end 113.84 35.915) (width 0.2) (layer "B.Cu") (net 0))
 (segment (start 97.8 50) (end 95.1 52.7) (width 0.2) (layer "B.Cu") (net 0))
 (segment (start 99.8 53) (end 101 53) (width 0.2) (layer "B.Cu") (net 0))
 (segment (start 99.7 67) (end 99.825 67) (width 0.2) (layer "B.Cu") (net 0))
 (segment (start 97.4 53) (end 96.4 54) (width 0.2) (layer "B.Cu") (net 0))
 (segment (start 114.485 53.36) (end 110.74 53.36) (width 0.2) (layer "B.Cu") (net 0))
 (segment (start 116 34) (end 117 35) (width 0.2) (layer "B.Cu") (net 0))
 (segment (start 109.475 50.625) (end 109.475 50) (width 0.2) (layer "B.Cu") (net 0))
 (segment (start 85.66 35.915) (end 84.085 35.915) (width 0.25) (layer "B.Cu") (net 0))
 (segment (start 109.475 42) (end 113.84 37.635) (width 0.2) (layer "B.Cu") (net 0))
 (segment (start 84.085 35.915) (end 83.3 36.7) (width 0.25) (layer "B.Cu") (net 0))
 (segment (start 108.675 36) (end 108.76 35.915) (width 0.2) (layer "B.Cu") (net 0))
 (segment (start 90.74 35.915) (end 90.74 39.265) (width 0.2) (layer "B.Cu") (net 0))
 (segment (start 99.825 67) (end 99.8625 66.9625) (width 0.2) (layer "B.Cu") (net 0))
 (segment (start 99.8 59.8) (end 101.475 58.125) (width 0.2) (layer "B.Cu") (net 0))
 (segment (start 102.24 35.915) (end 102.24 41.235) (width 0.2) (layer "B.Cu") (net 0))
 (segment (start 112.2 63.5) (end 113.4875 62.2125) (width 0.2) (layer "B.Cu") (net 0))
 (segment (start 108.76 35.915) (end 109.045 35.915) (width 0.2) (layer "B.Cu") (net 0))
 (segment (start 85.8 58.44) (end 85.8 61.5) (width 0.2) (layer "B.Cu") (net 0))
 (segment (start 115 34) (end 116 34) (width 0.2) (layer "B.Cu") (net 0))
 (segment (start 87.465 46.94) (end 90.525 50) (width 0.25) (layer "B.Cu") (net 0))
 (segment (start 83.4 49.3) (end 83.4 56.04) (width 0.25) (layer "B.Cu") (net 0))
 (segment (start 83.4 56.04) (end 85.8 58.44) (width 0.25) (layer "B.Cu") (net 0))
 (segment (start 101 53) (end 101.475 52.525) (width 0.2) (layer "B.Cu") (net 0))
 (segment (start 102.24 41.235) (end 101.475 42) (width 0.2) (layer "B.Cu") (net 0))
 (segment (start 117 35) (end 117 36) (width 0.2) (layer "B.Cu") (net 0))
 (segment (start 109.475 42.625) (end 109.475 42) (width 0.2) (layer "B.Cu") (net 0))
 (segment (start 112.2 65.7) (end 112.2 63.5) (width 0.2) (layer "B.Cu") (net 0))
 (segment (start 109.915 58.44) (end 113.785 58.44) (width 0.2) (layer "B.Cu") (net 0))
 (segment (start 91.4 54) (end 95.1 54) (width 0.25) (layer "B.Cu") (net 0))
 (segment (start 114.585 41.86) (end 115.6 40.845) (width 0.2) (layer "B.Cu") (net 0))
 (segment (start 92.5 58.5) (end 92.975 58.5) (width 0.2) (layer "B.Cu") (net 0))
 (segment (start 112.535 46.94) (end 113.785 46.94) (width 0.2) (layer "B.Cu") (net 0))
 (segment (start 99.8 53) (end 97.4 53) (width 0.2) (layer "B.Cu") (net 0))
 (segment (start 85.66 35.915) (end 85.66 34.16) (width 0.25) (layer "B.Cu") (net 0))
 (segment (start 117 36) (end 116.6 36) (width 0.2) (layer "B.Cu") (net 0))
 (segment (start 99.8625 66.9625) (end 109.6375 66.9625) (width 0.2) (layer "B.Cu") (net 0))
 (segment (start 97.04 66.54) (end 97.5 67) (width 0.2) (layer "B.Cu") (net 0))
 (segment (start 115.6 40.045) (end 115.6 40) (width 0.2) (layer "B.Cu") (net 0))
 (segment (start 114.9 34.1) (end 108.9 34.1) (width 0.2) (layer "B.Cu") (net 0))
 (segment (start 108.9 34.1) (end 108.76 34.24) (width 0.25) (layer "B.Cu") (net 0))
 (segment (start 98.525 58) (end 98.525 60.225) (width 0.2) (layer "B.Cu") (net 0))
 (segment (start 108.34 64.385) (end 109.655 65.7) (width 0.2) (layer "B.Cu") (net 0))
 (segment (start 101.475 58) (end 103.26 59.785) (width 0.2) (layer "B.Cu") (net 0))
 (segment (start 106.025 42.5) (end 106 42.475) (width 0.2) (layer "B.Cu") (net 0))
 (segment (start 106.525 57.575) (end 106.525 58) (width 0.2) (layer "B.Cu") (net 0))
 (segment (start 108.2 33.4) (end 108.9 34.1) (width 0.25) (layer "B.Cu") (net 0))
 (segment (start 96.4 54) (end 96.4 61.4) (width 0.2) (layer "B.Cu") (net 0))
 (segment (start 101.475 52.525) (end 101.475 50) (width 0.2) (layer "B.Cu") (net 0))
 (segment (start 109.475 50) (end 112.535 46.94) (width 0.2) (layer "B.Cu") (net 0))
 (segment (start 108.86 64.385) (end 107.86 64.385) (width 0.2) (layer "B.Cu") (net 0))
 (segment (start 99.9 44.075) (end 101.475 42.5) (width 0.2) (layer "B.Cu") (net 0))
 (segment (start 99.7 62.4) (end 99.7 67) (width 0.2) (layer "B.Cu") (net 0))
 (segment (start 83.44 49.3) (end 83.4 49.3) (width 0.25) (layer "B.Cu") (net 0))
 (segment (start 109.655 65.7) (end 110.9 65.7) (width 0.2) (layer "B.Cu") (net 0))
 (segment (start 113.3725 42.2725) (end 114.1725 42.2725) (width 0.2) (layer "B.Cu") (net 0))
 (segment (start 99.9 44.7) (end 99.9 44.075) (width 0.2) (layer "B.Cu") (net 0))
 (segment (start 98.6 60.3) (end 98.6 61.3) (width 0.2) (layer "B.Cu") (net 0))
 (segment (start 85.8 53.36) (end 89.335 53.36) (width 0.2) (layer "B.Cu") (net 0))
 (segment (start 93.475 42.925) (end 93.475 42) (width 0.2) (layer "B.Cu") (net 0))
 (segment (start 97.16 34.84) (end 97.16 34.34) (width 0.25) (layer "B.Cu") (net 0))
 (segment (start 91.96 62.44) (end 91.96 64.385) (width 0.2) (layer "B.Cu") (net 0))
 (segment (start 85.8 46.94) (end 83.44 49.3) (width 0.25) (layer "B.Cu") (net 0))
 (segment (start 107.3 44.8) (end 108.975 43.125) (width 0.2) (layer "B.Cu") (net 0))
 (segment (start 85.8 41.46) (end 86.56 41.46) (width 0.2) (layer "B.Cu") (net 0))
 (segment (start 93.975 48.875) (end 93.975 50.125) (width 0.2) (layer "B.Cu") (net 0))
 (segment (start 85.66 34.16) (end 96.74 34.16) (width 0.25) (layer "B.Cu") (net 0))
 (segment (start 98.6 61.3) (end 99.7 62.4) (width 0.2) (layer "B.Cu") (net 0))
 (segment (start 113.4875 62.2125) (end 116.1125 62.2125) (width 0.2) (layer "B.Cu") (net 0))
 (segment (start 114.9 34.1) (end 115 34) (width 0.2) (layer "B.Cu") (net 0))
 (segment (start 96.4 61.4) (end 93 61.4) (width 0.2) (layer "B.Cu") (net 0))
 (segment (start 87.8 63.5) (end 87.8 67) (width 0.2) (layer "B.Cu") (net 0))
 (segment (start 85.8 46.94) (end 87.465 46.94) (width 0.25) (layer "B.Cu") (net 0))
 (segment (start 110.9 65.7) (end 112.2 65.7) (width 0.2) (layer "B.Cu") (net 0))
 (segment (start 115.6 40.845) (end 115.6 40) (width 0.2) (layer "B.Cu") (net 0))
 (segment (start 109.6375 66.9625) (end 110.9 65.7) (width 0.2) (layer "B.Cu") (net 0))
 (segment (start 110.74 53.36) (end 106.525 57.575) (width 0.2) (layer "B.Cu") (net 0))
 (segment (start 106 42.475) (end 106 38.675) (width 0.2) (layer "B.Cu") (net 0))
 (segment (start 85.66 37.135) (end 85.66 35.915) (width 0.2) (layer "B.Cu") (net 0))
 (segment (start 85.8 61.5) (end 87.8 63.5) (width 0.2) (layer "B.Cu") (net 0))
 (segment (start 107.3 52.3) (end 108.975 50.625) (width 0.2) (layer "B.Cu") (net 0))
 (segment (start 98.525 37.28) (end 97.16 35.915) (width 0.2) (layer "B.Cu") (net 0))
 (segment (start 116.7 61.625) (end 116.7 55.575) (width 0.2) (layer "B.Cu") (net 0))
 (segment (start 97.16 34.06) (end 97.16 34.84) (width 0.25) (layer "B.Cu") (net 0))
 (segment (start 90.74 39.265) (end 93.475 42) (width 0.2) (layer "B.Cu") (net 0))
 (segment (start 98.525 42) (end 98.525 37.28) (width 0.2) (layer "B.Cu") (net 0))
 (segment (start 109.475 58) (end 109.915 58.44) (width 0.2) (layer "B.Cu") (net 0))
 (segment (start 92.8 44.6) (end 93.975 43.425) (width 0.2) (layer "B.Cu") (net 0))
 (segment (start 93 61.4) (end 91.96 62.44) (width 0.2) (layer "B.Cu") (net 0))
 (segment (start 90.525 50) (end 90.525 53.125) (width 0.25) (layer "B.Cu") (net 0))
 (segment (start 85.8 41.86) (end 85.8 41.46) (width 0.2) (layer "B.Cu") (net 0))
 (segment (start 83.3 36.7) (end 83.3 44.44) (width 0.25) (layer "B.Cu") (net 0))
 (segment (start 97.04 64.385) (end 97.04 66.54) (width 0.2) (layer "B.Cu") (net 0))
 (segment (start 90.525 42) (end 85.66 37.135) (width 0.2) (layer "B.Cu") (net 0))
 (segment (start 106.525 50) (end 106.525 49.12) (width 0.2) (layer "B.Cu") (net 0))
 (segment (start 116.7 55.575) (end 114.485 53.36) (width 0.2) (layer "B.Cu") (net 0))
 (segment (start 96.74 34.16) (end 97 33.9) (width 0.25) (layer "B.Cu") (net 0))
 (segment (start 83.3 44.44) (end 85.8 46.94) (width 0.25) (layer "B.Cu") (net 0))
 (segment (start 90.085 58.44) (end 90.525 58) (width 0.25) (layer "B.Cu") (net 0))
 (segment (start 116.1125 62.2125) (end 116.7 61.625) (width 0.2) (layer "B.Cu") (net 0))
 (segment (start 97 33.9) (end 97.16 34.06) (width 0.25) (layer "B.Cu") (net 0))
 (segment (start 97.16 34.34) (end 98.1 33.4) (width 0.25) (layer "B.Cu") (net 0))
 (segment (start 98.1 33.4) (end 108.2 33.4) (width 0.25) (layer "B.Cu") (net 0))
 (segment (start 107.0375 59.4375) (end 108.975 57.5) (width 0.2) (layer "B.Cu") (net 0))
 (segment (start 90.525 53.125) (end 91.4 54) (width 0.25) (layer "B.Cu") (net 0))
 (segment (start 115.6 40) (end 115.6 37) (width 0.2) (layer "B.Cu") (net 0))
 (segment (start 103.26 59.785) (end 103.26 64.385) (width 0.2) (layer "B.Cu") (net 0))
 (segment (start 114.1725 42.2725) (end 114.585 41.86) (width 0.2) (layer "B.Cu") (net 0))
 (segment (start 98.525 60.225) (end 98.6 60.3) (width 0.2) (layer "B.Cu") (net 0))
 (segment (start 85.8 58.44) (end 90.085 58.44) (width 0.25) (layer "B.Cu") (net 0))
 (segment (start 91.8 52.3) (end 93.5 52.3) (width 0.25) (layer "B.Cu") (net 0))
 (segment (start 98.525 50) (end 97.8 50) (width 0.2) (layer "B.Cu") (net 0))
 (segment (start 92.975 58.5) (end 93.975 57.5) (width 0.2) (layer "B.Cu") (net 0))
 (segment (start 108.76 34.24) (end 108.76 35.915) (width 0.25) (layer "B.Cu") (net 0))
 (segment (start 99.8 52.3) (end 99.8 53) (width 0.2) (layer "B.Cu") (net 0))
 (segment (start 93.975 51.825) (end 93.975 50) (width 0.25) (layer "B.Cu") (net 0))
 (segment (start 87.8 67) (end 97.5 67) (width 0.2) (layer "B.Cu") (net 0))
 (segment (start 109.045 35.915) (end 109.46 35.5) (width 0.2) (layer "B.Cu") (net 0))
 (segment (start 101.475 58.625) (end 101.475 58) (width 0.2) (layer "B.Cu") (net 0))
 (segment (start 106.525 49.12) (end 113.3725 42.2725) (width 0.2) (layer "B.Cu") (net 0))
 (segment (start 97.5 67) (end 99.7 67) (width 0.2) (layer "B.Cu") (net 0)))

